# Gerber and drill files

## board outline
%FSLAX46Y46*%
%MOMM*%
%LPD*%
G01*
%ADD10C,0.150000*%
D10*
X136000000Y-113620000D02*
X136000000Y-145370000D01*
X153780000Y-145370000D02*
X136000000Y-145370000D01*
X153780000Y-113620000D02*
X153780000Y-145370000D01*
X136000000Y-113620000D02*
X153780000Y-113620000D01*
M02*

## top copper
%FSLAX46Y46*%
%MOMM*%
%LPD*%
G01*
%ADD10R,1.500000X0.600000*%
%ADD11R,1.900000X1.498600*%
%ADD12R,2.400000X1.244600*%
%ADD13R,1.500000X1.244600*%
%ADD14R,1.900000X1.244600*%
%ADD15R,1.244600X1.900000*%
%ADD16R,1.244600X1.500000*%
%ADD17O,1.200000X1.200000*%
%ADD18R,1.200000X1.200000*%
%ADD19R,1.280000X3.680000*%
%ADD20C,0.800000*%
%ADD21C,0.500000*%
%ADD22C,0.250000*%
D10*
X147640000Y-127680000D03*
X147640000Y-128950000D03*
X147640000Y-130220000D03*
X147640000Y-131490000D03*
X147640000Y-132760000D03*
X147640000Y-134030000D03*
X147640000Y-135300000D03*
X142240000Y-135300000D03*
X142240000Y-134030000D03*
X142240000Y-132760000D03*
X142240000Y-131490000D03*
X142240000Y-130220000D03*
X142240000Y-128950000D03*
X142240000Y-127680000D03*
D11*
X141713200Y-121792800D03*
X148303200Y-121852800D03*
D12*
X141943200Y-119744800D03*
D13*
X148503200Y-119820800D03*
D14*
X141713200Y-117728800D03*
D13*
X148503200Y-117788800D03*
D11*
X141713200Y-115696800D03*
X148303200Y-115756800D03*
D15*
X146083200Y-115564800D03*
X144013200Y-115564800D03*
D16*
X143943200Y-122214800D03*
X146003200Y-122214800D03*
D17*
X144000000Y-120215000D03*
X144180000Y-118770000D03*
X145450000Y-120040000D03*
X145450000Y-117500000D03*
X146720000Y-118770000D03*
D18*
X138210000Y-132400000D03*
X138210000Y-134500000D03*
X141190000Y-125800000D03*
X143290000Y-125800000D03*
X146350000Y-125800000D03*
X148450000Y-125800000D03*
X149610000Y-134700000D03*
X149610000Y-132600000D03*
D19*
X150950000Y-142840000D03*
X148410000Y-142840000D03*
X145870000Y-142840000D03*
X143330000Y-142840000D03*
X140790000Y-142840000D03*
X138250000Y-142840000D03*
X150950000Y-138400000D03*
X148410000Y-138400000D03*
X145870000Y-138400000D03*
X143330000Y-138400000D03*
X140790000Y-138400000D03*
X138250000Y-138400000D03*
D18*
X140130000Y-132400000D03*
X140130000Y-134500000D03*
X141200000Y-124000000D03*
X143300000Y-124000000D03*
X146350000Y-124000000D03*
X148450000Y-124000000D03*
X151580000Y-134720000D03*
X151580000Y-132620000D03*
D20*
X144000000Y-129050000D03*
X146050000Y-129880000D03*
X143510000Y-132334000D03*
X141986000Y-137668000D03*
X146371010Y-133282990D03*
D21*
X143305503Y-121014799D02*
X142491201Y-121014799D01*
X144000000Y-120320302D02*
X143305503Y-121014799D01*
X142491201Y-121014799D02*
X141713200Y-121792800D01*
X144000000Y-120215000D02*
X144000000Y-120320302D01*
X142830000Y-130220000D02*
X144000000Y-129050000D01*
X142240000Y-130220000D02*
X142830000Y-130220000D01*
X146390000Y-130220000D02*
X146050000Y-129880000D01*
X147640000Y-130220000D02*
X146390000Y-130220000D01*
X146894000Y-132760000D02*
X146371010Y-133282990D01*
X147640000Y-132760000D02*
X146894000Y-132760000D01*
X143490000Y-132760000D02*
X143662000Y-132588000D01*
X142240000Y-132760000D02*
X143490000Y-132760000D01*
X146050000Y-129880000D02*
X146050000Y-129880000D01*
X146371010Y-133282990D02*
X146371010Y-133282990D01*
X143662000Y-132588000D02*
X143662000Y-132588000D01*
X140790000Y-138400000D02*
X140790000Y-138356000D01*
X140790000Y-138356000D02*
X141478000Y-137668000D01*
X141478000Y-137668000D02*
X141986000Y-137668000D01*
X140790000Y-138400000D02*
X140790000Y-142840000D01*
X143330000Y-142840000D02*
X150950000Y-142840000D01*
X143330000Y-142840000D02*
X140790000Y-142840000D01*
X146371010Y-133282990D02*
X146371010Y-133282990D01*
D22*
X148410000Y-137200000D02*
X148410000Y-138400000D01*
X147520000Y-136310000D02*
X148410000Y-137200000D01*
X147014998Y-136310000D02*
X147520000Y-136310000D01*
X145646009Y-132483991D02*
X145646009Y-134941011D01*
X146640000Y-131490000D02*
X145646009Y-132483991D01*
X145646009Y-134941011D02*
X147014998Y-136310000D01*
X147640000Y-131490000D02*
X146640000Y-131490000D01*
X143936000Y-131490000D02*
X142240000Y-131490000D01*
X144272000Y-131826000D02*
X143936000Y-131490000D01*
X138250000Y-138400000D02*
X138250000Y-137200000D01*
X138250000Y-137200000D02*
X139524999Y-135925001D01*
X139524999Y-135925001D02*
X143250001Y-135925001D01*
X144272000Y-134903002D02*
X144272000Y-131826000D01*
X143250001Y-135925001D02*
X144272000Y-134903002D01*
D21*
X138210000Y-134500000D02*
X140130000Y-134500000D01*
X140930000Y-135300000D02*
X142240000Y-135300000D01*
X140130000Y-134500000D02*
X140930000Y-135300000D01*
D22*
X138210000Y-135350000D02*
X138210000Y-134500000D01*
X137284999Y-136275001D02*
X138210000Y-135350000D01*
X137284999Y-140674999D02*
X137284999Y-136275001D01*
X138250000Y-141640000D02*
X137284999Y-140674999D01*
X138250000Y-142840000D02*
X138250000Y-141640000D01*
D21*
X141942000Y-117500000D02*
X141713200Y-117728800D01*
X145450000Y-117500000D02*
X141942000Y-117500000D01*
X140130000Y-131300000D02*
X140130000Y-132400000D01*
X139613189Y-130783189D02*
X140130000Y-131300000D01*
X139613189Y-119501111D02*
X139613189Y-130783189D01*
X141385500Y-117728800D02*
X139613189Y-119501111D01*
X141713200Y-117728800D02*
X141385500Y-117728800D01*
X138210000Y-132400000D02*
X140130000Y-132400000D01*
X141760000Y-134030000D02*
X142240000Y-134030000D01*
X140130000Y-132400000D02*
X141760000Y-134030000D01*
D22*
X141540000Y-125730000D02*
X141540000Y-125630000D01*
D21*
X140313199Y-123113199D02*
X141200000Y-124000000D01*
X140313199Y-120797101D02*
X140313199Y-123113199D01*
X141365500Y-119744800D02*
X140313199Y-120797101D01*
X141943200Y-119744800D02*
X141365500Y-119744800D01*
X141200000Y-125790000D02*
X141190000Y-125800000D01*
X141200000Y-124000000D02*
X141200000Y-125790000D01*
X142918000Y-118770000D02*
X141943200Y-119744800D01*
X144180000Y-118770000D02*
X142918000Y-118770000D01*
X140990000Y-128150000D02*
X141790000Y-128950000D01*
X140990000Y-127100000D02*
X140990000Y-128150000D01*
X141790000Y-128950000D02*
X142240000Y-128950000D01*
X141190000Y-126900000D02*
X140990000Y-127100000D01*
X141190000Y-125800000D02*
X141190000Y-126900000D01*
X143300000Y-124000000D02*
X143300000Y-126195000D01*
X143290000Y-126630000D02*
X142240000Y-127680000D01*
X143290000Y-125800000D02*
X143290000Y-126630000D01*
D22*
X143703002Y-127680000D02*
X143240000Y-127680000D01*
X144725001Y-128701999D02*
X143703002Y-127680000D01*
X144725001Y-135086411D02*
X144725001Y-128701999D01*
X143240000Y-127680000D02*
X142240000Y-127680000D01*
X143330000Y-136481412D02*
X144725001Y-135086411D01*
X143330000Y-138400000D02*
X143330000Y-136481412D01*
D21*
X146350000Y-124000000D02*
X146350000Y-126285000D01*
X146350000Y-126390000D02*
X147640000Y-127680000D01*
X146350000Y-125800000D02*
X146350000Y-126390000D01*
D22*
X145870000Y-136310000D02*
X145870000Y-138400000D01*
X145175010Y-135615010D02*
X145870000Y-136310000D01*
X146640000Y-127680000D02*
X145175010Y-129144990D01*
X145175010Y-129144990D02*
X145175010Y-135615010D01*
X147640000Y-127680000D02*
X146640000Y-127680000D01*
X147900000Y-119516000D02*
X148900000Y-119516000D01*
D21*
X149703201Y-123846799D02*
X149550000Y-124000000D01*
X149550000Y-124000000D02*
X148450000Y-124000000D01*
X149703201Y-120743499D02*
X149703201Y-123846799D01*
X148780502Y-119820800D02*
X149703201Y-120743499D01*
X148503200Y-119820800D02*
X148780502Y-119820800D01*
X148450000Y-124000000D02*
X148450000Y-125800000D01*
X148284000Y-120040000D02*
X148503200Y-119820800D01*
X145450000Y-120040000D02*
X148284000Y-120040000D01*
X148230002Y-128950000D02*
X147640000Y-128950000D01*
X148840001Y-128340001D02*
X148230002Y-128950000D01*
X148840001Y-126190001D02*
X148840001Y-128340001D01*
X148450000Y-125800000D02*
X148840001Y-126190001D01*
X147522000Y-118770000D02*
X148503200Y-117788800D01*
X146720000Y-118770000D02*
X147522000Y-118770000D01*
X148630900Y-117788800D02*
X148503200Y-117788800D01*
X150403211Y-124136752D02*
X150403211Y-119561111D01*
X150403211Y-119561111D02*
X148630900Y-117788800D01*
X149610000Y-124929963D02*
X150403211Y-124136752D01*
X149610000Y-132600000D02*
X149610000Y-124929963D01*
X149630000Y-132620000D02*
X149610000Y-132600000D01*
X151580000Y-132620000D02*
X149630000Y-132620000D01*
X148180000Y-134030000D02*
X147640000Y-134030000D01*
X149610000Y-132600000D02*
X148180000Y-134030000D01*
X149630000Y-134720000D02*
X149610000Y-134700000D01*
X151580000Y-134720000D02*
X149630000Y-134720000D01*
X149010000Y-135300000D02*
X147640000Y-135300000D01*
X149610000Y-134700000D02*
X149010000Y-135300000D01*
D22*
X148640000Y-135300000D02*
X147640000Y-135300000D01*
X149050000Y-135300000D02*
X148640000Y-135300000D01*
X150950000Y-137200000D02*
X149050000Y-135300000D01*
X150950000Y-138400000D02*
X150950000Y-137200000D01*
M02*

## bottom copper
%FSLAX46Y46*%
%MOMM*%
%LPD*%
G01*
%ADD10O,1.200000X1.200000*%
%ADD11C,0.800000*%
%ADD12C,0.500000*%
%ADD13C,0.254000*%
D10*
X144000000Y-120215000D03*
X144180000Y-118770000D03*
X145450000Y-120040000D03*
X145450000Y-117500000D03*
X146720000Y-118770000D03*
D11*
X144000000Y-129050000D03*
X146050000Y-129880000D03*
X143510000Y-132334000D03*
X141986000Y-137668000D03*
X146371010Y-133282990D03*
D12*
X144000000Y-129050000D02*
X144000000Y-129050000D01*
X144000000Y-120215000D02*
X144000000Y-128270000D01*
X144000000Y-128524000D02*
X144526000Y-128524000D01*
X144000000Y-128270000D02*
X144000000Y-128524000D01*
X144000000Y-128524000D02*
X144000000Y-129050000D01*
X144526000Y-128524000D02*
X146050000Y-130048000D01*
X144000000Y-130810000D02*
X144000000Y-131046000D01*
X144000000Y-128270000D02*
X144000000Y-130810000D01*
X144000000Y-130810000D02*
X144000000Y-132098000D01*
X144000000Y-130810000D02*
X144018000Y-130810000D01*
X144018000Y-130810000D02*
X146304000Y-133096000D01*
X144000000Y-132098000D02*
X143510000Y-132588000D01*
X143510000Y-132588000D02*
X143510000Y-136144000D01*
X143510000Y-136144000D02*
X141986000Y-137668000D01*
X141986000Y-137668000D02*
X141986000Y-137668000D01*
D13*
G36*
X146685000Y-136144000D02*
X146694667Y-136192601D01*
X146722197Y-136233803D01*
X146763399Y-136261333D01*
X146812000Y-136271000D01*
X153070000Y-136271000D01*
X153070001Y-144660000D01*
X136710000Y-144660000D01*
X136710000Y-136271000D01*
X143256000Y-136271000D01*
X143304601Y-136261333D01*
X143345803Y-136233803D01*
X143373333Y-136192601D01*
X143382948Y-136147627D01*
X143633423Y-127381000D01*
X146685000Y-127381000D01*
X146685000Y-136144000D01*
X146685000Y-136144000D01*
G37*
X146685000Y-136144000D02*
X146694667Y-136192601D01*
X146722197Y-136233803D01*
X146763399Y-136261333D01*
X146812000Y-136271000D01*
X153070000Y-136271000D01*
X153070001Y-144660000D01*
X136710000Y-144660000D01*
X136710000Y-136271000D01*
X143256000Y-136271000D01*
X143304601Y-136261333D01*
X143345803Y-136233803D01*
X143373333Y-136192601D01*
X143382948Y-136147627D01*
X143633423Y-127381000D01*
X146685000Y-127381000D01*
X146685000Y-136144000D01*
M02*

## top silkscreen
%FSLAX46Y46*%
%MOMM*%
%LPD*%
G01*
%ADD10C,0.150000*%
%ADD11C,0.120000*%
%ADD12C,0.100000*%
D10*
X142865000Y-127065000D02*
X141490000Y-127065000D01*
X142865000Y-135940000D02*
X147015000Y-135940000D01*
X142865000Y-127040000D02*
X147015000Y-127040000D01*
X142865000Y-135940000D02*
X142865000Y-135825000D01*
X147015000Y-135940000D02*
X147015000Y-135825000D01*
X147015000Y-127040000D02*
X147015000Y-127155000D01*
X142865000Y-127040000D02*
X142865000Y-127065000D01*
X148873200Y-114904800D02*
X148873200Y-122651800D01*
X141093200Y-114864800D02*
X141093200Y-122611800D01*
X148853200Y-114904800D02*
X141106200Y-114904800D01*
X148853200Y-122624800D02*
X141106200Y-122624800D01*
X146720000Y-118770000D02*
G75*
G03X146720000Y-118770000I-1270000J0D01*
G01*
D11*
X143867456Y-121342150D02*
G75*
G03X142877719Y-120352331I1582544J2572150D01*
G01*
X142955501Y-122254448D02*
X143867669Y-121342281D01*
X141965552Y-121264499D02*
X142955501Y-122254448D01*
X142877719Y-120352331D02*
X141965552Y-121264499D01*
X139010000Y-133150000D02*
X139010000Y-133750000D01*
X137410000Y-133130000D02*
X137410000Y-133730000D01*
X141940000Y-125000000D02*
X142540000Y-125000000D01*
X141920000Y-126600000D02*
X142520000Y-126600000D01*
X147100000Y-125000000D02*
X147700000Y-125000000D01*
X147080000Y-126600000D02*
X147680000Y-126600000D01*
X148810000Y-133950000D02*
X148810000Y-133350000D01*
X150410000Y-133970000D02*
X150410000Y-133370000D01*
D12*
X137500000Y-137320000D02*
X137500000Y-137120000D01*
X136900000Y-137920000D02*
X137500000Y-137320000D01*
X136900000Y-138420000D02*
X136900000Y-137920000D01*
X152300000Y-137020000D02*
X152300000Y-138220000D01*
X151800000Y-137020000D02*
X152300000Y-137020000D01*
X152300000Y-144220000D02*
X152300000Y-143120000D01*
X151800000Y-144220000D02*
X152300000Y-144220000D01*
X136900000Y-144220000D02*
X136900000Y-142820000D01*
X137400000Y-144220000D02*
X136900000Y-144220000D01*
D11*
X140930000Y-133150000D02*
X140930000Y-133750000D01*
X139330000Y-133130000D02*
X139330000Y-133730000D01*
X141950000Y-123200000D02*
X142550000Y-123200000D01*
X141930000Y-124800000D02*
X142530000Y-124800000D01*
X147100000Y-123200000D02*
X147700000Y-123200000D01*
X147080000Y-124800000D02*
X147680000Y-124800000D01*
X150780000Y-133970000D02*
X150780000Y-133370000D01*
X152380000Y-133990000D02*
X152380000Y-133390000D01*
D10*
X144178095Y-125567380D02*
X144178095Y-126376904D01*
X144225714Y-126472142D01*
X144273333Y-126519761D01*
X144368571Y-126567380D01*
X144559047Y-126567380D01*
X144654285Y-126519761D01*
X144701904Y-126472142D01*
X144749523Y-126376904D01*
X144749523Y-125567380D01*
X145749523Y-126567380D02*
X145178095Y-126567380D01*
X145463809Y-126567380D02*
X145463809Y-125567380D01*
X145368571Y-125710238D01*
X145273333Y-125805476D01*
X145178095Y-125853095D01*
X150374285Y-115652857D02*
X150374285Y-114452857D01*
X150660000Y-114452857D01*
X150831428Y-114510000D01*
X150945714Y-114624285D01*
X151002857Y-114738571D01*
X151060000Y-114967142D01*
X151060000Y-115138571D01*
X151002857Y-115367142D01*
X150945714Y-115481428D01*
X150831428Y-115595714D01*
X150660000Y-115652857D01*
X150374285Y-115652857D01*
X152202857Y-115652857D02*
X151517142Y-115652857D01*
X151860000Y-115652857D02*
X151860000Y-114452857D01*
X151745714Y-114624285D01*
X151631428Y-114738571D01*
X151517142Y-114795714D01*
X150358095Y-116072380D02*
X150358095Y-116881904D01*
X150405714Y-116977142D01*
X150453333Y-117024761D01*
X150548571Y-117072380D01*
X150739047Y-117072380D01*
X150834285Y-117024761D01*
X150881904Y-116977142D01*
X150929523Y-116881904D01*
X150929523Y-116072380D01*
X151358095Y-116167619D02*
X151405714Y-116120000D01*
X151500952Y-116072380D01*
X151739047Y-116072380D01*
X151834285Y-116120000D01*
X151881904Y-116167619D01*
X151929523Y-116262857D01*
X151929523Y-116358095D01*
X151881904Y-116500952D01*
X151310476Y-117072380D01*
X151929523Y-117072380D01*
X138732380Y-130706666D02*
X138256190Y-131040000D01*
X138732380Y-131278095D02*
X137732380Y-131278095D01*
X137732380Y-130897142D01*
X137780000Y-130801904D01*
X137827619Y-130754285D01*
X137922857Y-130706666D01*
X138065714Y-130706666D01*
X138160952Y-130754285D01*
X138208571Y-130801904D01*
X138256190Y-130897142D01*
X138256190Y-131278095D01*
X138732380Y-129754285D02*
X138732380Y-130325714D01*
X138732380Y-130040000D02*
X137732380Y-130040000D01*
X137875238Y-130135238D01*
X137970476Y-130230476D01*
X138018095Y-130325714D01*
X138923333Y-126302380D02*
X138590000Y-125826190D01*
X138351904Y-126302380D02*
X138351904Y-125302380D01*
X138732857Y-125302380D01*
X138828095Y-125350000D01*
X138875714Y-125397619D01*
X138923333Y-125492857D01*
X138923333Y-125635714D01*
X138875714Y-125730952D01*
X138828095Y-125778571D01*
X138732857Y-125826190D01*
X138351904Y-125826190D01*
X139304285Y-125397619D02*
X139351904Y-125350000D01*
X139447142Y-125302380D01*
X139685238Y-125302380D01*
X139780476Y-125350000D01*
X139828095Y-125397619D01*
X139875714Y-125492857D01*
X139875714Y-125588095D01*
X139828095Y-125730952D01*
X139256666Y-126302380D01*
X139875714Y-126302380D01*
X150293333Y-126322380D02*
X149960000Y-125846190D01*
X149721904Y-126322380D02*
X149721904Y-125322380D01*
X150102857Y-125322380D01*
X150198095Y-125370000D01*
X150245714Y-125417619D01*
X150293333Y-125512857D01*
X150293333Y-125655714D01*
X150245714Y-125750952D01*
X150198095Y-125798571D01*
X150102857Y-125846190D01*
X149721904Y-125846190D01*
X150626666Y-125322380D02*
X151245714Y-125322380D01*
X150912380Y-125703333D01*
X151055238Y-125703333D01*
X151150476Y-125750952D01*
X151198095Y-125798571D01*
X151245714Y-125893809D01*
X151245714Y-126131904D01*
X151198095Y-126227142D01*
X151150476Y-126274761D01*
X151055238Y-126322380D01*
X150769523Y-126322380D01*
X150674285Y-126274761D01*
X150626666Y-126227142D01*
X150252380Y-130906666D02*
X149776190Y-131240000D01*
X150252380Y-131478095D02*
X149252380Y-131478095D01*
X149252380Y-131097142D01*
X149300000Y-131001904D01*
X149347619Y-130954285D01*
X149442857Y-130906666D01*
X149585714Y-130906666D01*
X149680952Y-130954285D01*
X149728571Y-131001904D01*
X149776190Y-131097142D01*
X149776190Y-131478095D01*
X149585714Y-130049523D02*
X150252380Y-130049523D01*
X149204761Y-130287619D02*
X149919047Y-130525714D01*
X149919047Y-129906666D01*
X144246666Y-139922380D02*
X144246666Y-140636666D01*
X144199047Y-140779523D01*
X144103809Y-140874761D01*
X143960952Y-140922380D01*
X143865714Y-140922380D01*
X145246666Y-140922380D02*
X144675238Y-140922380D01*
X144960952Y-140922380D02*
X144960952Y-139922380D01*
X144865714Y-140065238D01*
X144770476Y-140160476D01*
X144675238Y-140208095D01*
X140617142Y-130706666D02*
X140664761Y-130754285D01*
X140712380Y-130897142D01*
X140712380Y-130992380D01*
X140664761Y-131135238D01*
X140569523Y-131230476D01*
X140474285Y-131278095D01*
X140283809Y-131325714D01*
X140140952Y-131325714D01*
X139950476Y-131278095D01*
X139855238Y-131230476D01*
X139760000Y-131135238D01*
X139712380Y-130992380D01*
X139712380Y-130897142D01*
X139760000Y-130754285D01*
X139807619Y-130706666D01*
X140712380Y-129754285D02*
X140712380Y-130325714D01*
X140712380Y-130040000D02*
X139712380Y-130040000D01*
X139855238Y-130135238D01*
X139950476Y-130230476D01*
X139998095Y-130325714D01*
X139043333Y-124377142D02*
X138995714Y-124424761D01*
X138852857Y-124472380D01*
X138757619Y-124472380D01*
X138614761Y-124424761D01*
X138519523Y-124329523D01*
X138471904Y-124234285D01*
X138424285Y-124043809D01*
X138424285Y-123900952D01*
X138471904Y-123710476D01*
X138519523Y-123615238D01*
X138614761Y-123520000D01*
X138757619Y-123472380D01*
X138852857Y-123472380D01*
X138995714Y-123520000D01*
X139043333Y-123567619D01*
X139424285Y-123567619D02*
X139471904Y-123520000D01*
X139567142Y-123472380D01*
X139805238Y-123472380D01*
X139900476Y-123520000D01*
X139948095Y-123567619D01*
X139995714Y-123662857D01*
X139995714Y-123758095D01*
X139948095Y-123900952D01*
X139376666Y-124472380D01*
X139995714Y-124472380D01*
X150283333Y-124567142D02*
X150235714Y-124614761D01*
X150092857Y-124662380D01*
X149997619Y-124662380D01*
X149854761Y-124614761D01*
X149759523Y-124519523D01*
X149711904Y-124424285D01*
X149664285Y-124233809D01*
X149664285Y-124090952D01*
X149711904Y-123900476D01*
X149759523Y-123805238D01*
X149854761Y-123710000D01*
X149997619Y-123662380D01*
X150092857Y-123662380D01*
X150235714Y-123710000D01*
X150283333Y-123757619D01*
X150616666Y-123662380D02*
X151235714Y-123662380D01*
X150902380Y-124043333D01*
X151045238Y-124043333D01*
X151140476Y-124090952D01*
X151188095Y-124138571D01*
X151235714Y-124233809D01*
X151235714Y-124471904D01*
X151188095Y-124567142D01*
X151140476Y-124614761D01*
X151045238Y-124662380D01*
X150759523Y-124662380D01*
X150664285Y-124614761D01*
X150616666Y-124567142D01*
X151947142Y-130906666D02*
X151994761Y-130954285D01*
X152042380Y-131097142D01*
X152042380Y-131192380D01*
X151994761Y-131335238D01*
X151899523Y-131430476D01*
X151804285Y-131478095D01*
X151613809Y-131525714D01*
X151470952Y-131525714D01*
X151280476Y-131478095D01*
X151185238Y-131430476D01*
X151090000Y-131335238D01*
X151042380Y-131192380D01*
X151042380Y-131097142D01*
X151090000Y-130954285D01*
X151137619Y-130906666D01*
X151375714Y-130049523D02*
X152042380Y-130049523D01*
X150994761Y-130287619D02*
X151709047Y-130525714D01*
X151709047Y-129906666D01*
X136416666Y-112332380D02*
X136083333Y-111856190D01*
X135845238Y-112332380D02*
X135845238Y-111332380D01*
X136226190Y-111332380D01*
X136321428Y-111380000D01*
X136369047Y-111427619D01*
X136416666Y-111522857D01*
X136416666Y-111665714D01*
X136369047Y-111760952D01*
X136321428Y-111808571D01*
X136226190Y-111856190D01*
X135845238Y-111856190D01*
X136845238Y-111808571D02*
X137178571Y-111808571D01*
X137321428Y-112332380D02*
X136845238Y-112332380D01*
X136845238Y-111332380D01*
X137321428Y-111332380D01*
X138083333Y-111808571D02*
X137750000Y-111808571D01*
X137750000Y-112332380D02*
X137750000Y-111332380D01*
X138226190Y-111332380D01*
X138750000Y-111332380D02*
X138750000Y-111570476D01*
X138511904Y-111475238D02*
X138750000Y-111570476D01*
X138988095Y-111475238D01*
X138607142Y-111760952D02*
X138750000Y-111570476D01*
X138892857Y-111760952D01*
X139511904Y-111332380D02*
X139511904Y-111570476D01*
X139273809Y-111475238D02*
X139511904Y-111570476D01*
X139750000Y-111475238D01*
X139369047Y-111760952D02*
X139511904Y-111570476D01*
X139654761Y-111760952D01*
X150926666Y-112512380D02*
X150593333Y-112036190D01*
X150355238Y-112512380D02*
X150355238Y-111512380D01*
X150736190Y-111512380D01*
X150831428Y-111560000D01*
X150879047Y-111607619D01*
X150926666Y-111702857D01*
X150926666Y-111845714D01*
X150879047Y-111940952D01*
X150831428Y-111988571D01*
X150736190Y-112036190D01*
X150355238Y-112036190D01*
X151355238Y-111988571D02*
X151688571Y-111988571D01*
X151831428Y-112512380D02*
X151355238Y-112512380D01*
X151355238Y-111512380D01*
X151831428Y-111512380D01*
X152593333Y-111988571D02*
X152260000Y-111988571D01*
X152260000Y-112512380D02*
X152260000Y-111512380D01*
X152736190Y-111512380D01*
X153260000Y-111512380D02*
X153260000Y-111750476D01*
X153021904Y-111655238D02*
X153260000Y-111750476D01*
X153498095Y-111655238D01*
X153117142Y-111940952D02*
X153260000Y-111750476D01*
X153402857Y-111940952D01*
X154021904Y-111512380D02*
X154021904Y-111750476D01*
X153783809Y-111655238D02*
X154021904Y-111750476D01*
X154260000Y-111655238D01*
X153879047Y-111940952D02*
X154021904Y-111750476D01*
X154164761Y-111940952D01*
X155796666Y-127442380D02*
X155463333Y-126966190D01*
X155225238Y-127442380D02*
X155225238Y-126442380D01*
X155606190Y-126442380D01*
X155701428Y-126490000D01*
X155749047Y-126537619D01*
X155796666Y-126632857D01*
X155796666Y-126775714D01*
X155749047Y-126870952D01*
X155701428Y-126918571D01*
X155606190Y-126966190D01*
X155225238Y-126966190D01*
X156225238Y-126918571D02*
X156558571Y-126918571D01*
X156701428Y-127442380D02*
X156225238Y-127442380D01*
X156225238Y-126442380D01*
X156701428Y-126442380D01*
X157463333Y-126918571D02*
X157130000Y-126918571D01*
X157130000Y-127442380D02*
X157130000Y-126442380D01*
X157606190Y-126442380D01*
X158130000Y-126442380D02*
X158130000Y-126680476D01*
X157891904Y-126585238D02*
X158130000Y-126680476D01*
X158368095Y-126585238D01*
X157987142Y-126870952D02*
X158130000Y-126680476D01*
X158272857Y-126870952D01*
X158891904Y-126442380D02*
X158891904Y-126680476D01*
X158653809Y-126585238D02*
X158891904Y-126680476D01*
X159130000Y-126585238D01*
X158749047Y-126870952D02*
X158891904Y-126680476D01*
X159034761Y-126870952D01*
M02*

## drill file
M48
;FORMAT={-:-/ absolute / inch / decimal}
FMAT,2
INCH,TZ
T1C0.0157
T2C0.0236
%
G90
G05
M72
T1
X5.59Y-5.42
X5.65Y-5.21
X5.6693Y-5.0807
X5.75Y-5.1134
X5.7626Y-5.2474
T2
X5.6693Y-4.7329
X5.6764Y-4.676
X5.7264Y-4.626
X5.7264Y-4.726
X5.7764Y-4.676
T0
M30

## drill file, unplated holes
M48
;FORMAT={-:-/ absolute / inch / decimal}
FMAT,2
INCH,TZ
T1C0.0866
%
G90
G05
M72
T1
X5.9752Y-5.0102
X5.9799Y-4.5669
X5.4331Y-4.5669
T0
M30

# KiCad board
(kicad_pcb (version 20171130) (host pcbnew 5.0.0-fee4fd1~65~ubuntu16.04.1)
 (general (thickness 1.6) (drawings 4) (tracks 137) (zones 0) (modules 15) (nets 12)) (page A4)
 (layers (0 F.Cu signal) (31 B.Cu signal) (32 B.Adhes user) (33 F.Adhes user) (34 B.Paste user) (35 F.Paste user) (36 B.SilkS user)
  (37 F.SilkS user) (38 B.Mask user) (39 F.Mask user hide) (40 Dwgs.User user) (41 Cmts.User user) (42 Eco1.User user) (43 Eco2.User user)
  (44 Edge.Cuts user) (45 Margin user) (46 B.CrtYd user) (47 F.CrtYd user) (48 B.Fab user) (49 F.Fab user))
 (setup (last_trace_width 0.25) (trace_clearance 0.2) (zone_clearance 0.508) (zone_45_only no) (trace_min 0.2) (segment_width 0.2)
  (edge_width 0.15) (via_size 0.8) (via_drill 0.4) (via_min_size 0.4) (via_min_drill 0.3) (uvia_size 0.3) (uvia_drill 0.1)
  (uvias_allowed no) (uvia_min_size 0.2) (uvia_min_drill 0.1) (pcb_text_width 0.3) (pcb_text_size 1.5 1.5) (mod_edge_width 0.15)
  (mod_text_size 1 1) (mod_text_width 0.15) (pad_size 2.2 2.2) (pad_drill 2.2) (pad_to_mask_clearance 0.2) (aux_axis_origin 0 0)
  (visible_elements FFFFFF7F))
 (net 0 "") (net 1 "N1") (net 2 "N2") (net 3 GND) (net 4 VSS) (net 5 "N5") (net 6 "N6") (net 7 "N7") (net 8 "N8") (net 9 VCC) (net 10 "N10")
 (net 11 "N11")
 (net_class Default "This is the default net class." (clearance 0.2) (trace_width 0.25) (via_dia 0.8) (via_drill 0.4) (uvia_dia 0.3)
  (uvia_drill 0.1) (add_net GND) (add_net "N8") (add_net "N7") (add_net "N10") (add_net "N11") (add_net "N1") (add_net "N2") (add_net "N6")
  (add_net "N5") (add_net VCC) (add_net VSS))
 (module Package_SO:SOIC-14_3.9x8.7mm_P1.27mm (layer F.Cu) (at 144.94 131.49)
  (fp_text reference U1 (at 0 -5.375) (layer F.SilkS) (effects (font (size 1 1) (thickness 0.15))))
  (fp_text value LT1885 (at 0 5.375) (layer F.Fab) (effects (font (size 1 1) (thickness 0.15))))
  (fp_line (start -2.075 -4.425) (end -3.45 -4.425) (layer F.SilkS) (width 0.15))
  (fp_line (start -2.075 4.45) (end 2.075 4.45) (layer F.SilkS) (width 0.15))
  (fp_line (start -2.075 -4.45) (end 2.075 -4.45) (layer F.SilkS) (width 0.15))
  (fp_line (start -2.075 4.45) (end -2.075 4.335) (layer F.SilkS) (width 0.15))
  (fp_line (start 2.075 4.45) (end 2.075 4.335) (layer F.SilkS) (width 0.15))
  (fp_line (start 2.075 -4.45) (end 2.075 -4.335) (layer F.SilkS) (width 0.15))
  (fp_line (start -2.075 -4.45) (end -2.075 -4.425) (layer F.SilkS) (width 0.15))
  (pad 14 smd rect (at 2.7 -3.81) (size 1.5 0.6) (layers F.Cu F.Paste F.Mask) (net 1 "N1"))
  (pad 13 smd rect (at 2.7 -2.54) (size 1.5 0.6) (layers F.Cu F.Paste F.Mask) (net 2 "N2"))
  (pad 12 smd rect (at 2.7 -1.27) (size 1.5 0.6) (layers F.Cu F.Paste F.Mask) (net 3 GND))
  (pad 11 smd rect (at 2.7 0) (size 1.5 0.6) (layers F.Cu F.Paste F.Mask) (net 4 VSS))
  (pad 10 smd rect (at 2.7 1.27) (size 1.5 0.6) (layers F.Cu F.Paste F.Mask) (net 3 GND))
  (pad 9 smd rect (at 2.7 2.54) (size 1.5 0.6) (layers F.Cu F.Paste F.Mask) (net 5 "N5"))
  (pad 8 smd rect (at 2.7 3.81) (size 1.5 0.6) (layers F.Cu F.Paste F.Mask) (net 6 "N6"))
  (pad 7 smd rect (at -2.7 3.81) (size 1.5 0.6) (layers F.Cu F.Paste F.Mask) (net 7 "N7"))
  (pad 6 smd rect (at -2.7 2.54) (size 1.5 0.6) (layers F.Cu F.Paste F.Mask) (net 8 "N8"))
  (pad 5 smd rect (at -2.7 1.27) (size 1.5 0.6) (layers F.Cu F.Paste F.Mask) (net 3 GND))
  (pad 4 smd rect (at -2.7 0) (size 1.5 0.6) (layers F.Cu F.Paste F.Mask) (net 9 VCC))
  (pad 3 smd rect (at -2.7 -1.27) (size 1.5 0.6) (layers F.Cu F.Paste F.Mask) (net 3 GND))
  (pad 2 smd rect (at -2.7 -2.54) (size 1.5 0.6) (layers F.Cu F.Paste F.Mask) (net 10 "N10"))
  (pad 1 smd rect (at -2.7 -3.81) (size 1.5 0.6) (layers F.Cu F.Paste F.Mask) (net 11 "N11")))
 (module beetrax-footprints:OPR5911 (layer F.Cu) (at 148.7932 117.1448 270)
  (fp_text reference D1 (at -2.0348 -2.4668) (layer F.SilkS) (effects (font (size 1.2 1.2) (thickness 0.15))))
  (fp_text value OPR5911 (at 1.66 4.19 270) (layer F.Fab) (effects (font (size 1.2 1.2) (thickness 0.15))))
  (fp_line (start -2.24 -0.08) (end 5.507 -0.08) (layer F.SilkS) (width 0.15))
  (fp_line (start -2.28 7.7) (end 5.467 7.7) (layer F.SilkS) (width 0.15))
  (fp_line (start -2.24 -0.06) (end -2.24 7.687) (layer F.SilkS) (width 0.15))
  (fp_line (start 5.48 -0.06) (end 5.48 7.687) (layer F.SilkS) (width 0.15))
  (pad 2 smd rect (at 4.648 7.08 270) (size 1.4986 1.9) (layers F.Cu F.Paste F.Mask) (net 3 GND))
  (pad 5 smd rect (at 4.708 0.49 270) (size 1.4986 1.9) (layers F.Cu F.Paste F.Mask))
  (pad 1 smd rect (at 2.6 6.85 270) (size 1.2446 2.4) (layers F.Cu F.Paste F.Mask) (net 10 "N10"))
  (pad 6 smd rect (at 2.676 0.29 270) (size 1.2446 1.5) (layers F.Cu F.Paste F.Mask) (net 2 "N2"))
  (pad 12 smd rect (at 0.584 7.08 270) (size 1.2446 1.9) (layers F.Cu F.Paste F.Mask) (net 8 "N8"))
  (pad 7 smd rect (at 0.644 0.29 270) (size 1.2446 1.5) (layers F.Cu F.Paste F.Mask) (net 5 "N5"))
  (pad 11 smd rect (at -1.448 7.08 270) (size 1.4986 1.9) (layers F.Cu F.Paste F.Mask))
  (pad 8 smd rect (at -1.388 0.49 270) (size 1.4986 1.9) (layers F.Cu F.Paste F.Mask))
  (pad 9 smd rect (at -1.58 2.71 270) (size 1.9 1.2446) (layers F.Cu F.Paste F.Mask))
  (pad 10 smd rect (at -1.58 4.78 270) (size 1.9 1.2446) (layers F.Cu F.Paste F.Mask))
  (pad 3 smd rect (at 5.07 4.85 270) (size 1.5 1.2446) (layers F.Cu F.Paste F.Mask))
  (pad 4 smd rect (at 5.07 2.79 270) (size 1.5 1.2446) (layers F.Cu F.Paste F.Mask)))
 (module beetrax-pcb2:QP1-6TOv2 (layer F.Cu) (at 145.45 120.04 90)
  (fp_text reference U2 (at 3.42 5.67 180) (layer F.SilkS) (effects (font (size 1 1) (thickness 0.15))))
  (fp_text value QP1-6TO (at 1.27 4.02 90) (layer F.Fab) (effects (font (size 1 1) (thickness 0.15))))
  (fp_circle (center 1.27 0) (end 1.27 1.27) (layer F.SilkS) (width 0.15))
  (fp_arc (start 1.27 0) (end -0.312331 -2.572281) (angle 333.2) (layer F.SilkS) (width 0.12))
  (fp_line (start -2.214448 -2.494499) (end -1.302281 -1.582331) (layer F.SilkS) (width 0.12))
  (fp_line (start -1.224499 -3.484448) (end -2.214448 -2.494499) (layer F.SilkS) (width 0.12))
  (fp_line (start -0.312331 -2.572281) (end -1.224499 -3.484448) (layer F.SilkS) (width 0.12))
  (pad 5 thru_hole oval (at -0.175 -1.45 90) (size 1.2 1.2) (drill 0.6) (layers *.Cu *.Mask) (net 3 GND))
  (pad 1 thru_hole oval (at 1.27 -1.27 90) (size 1.2 1.2) (drill 0.6) (layers *.Cu *.Mask) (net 10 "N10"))
  (pad 4 thru_hole oval (at 0 0 90) (size 1.2 1.2) (drill 0.6) (layers *.Cu *.Mask) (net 2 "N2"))
  (pad 2 thru_hole oval (at 2.54 0 90) (size 1.2 1.2) (drill 0.6) (layers *.Cu *.Mask) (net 8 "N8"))
  (pad 3 thru_hole oval (at 1.27 1.27 90) (size 1.2 1.2) (drill 0.6) (layers *.Cu *.Mask) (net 5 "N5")))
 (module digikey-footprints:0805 (layer F.Cu) (at 138.21 133.45 270)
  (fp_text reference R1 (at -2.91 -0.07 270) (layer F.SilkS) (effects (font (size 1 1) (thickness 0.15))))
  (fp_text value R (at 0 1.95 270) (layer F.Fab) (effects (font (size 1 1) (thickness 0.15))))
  (fp_line (start -0.3 -0.8) (end 0.3 -0.8) (layer F.SilkS) (width 0.12))
  (fp_line (start -0.32 0.8) (end 0.28 0.8) (layer F.SilkS) (width 0.12))
  (pad 1 smd rect (at -1.05 0 270) (size 1.2 1.2) (layers F.Cu F.Paste F.Mask) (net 8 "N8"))
  (pad 2 smd rect (at 1.05 0 270) (size 1.2 1.2) (layers F.Cu F.Paste F.Mask) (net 7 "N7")))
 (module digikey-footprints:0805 (layer F.Cu) (at 142.24 125.8)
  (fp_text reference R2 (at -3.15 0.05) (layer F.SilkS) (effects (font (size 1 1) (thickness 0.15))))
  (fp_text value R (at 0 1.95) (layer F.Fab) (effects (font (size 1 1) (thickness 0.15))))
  (fp_line (start -0.3 -0.8) (end 0.3 -0.8) (layer F.SilkS) (width 0.12))
  (fp_line (start -0.32 0.8) (end 0.28 0.8) (layer F.SilkS) (width 0.12))
  (pad 1 smd rect (at -1.05 0) (size 1.2 1.2) (layers F.Cu F.Paste F.Mask) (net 10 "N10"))
  (pad 2 smd rect (at 1.05 0) (size 1.2 1.2) (layers F.Cu F.Paste F.Mask) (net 11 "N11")))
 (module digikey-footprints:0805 (layer F.Cu) (at 147.4 125.8)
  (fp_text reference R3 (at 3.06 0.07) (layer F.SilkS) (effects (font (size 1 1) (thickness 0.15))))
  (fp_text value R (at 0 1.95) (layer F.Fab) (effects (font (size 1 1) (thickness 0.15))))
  (fp_line (start -0.3 -0.8) (end 0.3 -0.8) (layer F.SilkS) (width 0.12))
  (fp_line (start -0.32 0.8) (end 0.28 0.8) (layer F.SilkS) (width 0.12))
  (pad 1 smd rect (at -1.05 0) (size 1.2 1.2) (layers F.Cu F.Paste F.Mask) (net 1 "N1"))
  (pad 2 smd rect (at 1.05 0) (size 1.2 1.2) (layers F.Cu F.Paste F.Mask) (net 2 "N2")))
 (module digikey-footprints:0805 (layer F.Cu) (at 149.61 133.65 90)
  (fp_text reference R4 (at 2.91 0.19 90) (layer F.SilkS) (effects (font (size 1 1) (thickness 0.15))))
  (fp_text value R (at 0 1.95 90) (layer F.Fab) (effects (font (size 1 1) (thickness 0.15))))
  (fp_line (start -0.3 -0.8) (end 0.3 -0.8) (layer F.SilkS) (width 0.12))
  (fp_line (start -0.32 0.8) (end 0.28 0.8) (layer F.SilkS) (width 0.12))
  (pad 1 smd rect (at -1.05 0 90) (size 1.2 1.2) (layers F.Cu F.Paste F.Mask) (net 6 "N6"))
  (pad 2 smd rect (at 1.05 0 90) (size 1.2 1.2) (layers F.Cu F.Paste F.Mask) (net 5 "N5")))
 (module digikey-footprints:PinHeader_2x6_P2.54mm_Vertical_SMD (layer F.Cu) (at 144.6 140.62)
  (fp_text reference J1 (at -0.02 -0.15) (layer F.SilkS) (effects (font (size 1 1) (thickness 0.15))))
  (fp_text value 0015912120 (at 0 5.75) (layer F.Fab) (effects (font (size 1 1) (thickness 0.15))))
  (fp_line (start -7.1 -3.3) (end -7.1 -3.5) (layer F.SilkS) (width 0.1))
  (fp_line (start -7.7 -2.7) (end -7.1 -3.3) (layer F.SilkS) (width 0.1))
  (fp_line (start -7.7 -2.2) (end -7.7 -2.7) (layer F.SilkS) (width 0.1))
  (fp_line (start 7.7 -3.6) (end 7.7 -2.4) (layer F.SilkS) (width 0.1))
  (fp_line (start 7.2 -3.6) (end 7.7 -3.6) (layer F.SilkS) (width 0.1))
  (fp_line (start 7.7 3.6) (end 7.7 2.5) (layer F.SilkS) (width 0.1))
  (fp_line (start 7.2 3.6) (end 7.7 3.6) (layer F.SilkS) (width 0.1))
  (fp_line (start -7.7 3.6) (end -7.7 2.2) (layer F.SilkS) (width 0.1))
  (fp_line (start -7.2 3.6) (end -7.7 3.6) (layer F.SilkS) (width 0.1))
  (pad 12 smd rect (at 6.35 2.22) (size 1.28 3.68) (layers F.Cu F.Paste F.Mask) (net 3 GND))
  (pad 11 smd rect (at 3.81 2.22) (size 1.28 3.68) (layers F.Cu F.Paste F.Mask) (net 3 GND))
  (pad 10 smd rect (at 1.27 2.22) (size 1.28 3.68) (layers F.Cu F.Paste F.Mask) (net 3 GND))
  (pad 9 smd rect (at -1.27 2.22) (size 1.28 3.68) (layers F.Cu F.Paste F.Mask) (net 3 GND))
  (pad 8 smd rect (at -3.81 2.22) (size 1.28 3.68) (layers F.Cu F.Paste F.Mask) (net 3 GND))
  (pad 7 smd rect (at -6.35 2.22) (size 1.28 3.68) (layers F.Cu F.Paste F.Mask) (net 7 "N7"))
  (pad 6 smd rect (at 6.35 -2.22) (size 1.28 3.68) (layers F.Cu F.Paste F.Mask) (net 6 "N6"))
  (pad 5 smd rect (at 3.81 -2.22) (size 1.28 3.68) (layers F.Cu F.Paste F.Mask) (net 4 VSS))
  (pad 4 smd rect (at 1.27 -2.22) (size 1.28 3.68) (layers F.Cu F.Paste F.Mask) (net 1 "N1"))
  (pad 3 smd rect (at -1.27 -2.22) (size 1.28 3.68) (layers F.Cu F.Paste F.Mask) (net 11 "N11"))
  (pad 2 smd rect (at -3.81 -2.22) (size 1.28 3.68) (layers F.Cu F.Paste F.Mask) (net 3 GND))
  (pad 1 smd rect (at -6.35 -2.22) (size 1.28 3.68) (layers F.Cu F.Paste F.Mask) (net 9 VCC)))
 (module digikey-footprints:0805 (layer F.Cu) (at 140.13 133.45 270)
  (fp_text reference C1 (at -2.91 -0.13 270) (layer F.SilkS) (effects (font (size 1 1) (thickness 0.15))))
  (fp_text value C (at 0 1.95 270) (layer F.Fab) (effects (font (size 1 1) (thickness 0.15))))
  (fp_line (start -0.3 -0.8) (end 0.3 -0.8) (layer F.SilkS) (width 0.12))
  (fp_line (start -0.32 0.8) (end 0.28 0.8) (layer F.SilkS) (width 0.12))
  (pad 1 smd rect (at -1.05 0 270) (size 1.2 1.2) (layers F.Cu F.Paste F.Mask) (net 8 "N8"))
  (pad 2 smd rect (at 1.05 0 270) (size 1.2 1.2) (layers F.Cu F.Paste F.Mask) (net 7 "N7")))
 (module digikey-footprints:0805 (layer F.Cu) (at 142.25 124)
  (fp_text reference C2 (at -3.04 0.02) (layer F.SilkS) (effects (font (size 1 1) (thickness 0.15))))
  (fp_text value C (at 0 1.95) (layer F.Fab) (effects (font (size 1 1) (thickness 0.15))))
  (fp_line (start -0.3 -0.8) (end 0.3 -0.8) (layer F.SilkS) (width 0.12))
  (fp_line (start -0.32 0.8) (end 0.28 0.8) (layer F.SilkS) (width 0.12))
  (pad 1 smd rect (at -1.05 0) (size 1.2 1.2) (layers F.Cu F.Paste F.Mask) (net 10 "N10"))
  (pad 2 smd rect (at 1.05 0) (size 1.2 1.2) (layers F.Cu F.Paste F.Mask) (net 11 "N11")))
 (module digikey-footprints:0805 (layer F.Cu) (at 147.4 124)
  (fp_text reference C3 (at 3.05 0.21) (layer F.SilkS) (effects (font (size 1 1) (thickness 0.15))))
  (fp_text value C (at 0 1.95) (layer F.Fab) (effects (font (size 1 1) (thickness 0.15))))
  (fp_line (start -0.3 -0.8) (end 0.3 -0.8) (layer F.SilkS) (width 0.12))
  (fp_line (start -0.32 0.8) (end 0.28 0.8) (layer F.SilkS) (width 0.12))
  (pad 1 smd rect (at -1.05 0) (size 1.2 1.2) (layers F.Cu F.Paste F.Mask) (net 1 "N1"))
  (pad 2 smd rect (at 1.05 0) (size 1.2 1.2) (layers F.Cu F.Paste F.Mask) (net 2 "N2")))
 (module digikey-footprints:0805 (layer F.Cu) (at 151.58 133.67 90)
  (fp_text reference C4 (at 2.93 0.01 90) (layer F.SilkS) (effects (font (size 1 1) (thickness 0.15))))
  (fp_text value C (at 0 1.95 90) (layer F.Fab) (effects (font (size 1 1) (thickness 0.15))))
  (fp_line (start -0.3 -0.8) (end 0.3 -0.8) (layer F.SilkS) (width 0.12))
  (fp_line (start -0.32 0.8) (end 0.28 0.8) (layer F.SilkS) (width 0.12))
  (pad 1 smd rect (at -1.05 0 90) (size 1.2 1.2) (layers F.Cu F.Paste F.Mask) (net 6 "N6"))
  (pad 2 smd rect (at 1.05 0 90) (size 1.2 1.2) (layers F.Cu F.Paste F.Mask) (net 5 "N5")))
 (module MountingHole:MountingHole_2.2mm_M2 (layer F.Cu) (at 138 116)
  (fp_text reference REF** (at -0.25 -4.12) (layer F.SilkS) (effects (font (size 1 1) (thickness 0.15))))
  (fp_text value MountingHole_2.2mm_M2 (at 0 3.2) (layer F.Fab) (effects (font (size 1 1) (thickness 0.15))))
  (pad 1 np_thru_hole circle (at 0 0) (size 2.2 2.2) (drill 2.2) (layers *.Cu *.Mask)))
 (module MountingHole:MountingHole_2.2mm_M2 (layer F.Cu) (at 151.89 116)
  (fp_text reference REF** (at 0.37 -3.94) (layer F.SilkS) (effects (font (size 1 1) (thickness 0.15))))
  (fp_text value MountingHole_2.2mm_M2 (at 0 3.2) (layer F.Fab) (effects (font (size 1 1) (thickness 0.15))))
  (pad 1 np_thru_hole circle (at 0 0) (size 2.2 2.2) (drill 2.2) (layers *.Cu *.Mask)))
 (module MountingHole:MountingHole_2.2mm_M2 (layer F.Cu) (at 151.77 127.26)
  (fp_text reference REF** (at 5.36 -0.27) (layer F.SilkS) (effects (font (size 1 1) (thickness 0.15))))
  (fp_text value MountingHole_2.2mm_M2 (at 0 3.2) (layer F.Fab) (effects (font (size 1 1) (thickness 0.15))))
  (pad 1 np_thru_hole circle (at 0 0) (size 2.2 2.2) (drill 2.2) (layers *.Cu *.Mask)))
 (gr_line (start 136 113.62) (end 136 145.37) (layer Edge.Cuts) (width 0.15))
 (gr_line (start 153.78 145.37) (end 136 145.37) (layer Edge.Cuts) (width 0.15))
 (gr_line (start 153.78 113.62) (end 153.78 145.37) (layer Edge.Cuts) (width 0.15))
 (gr_line (start 136 113.62) (end 153.78 113.62) (layer Edge.Cuts) (width 0.15))
 (segment (start 143.305503 121.014799) (end 142.491201 121.014799) (width 0.5) (layer F.Cu) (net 3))
 (segment (start 144 120.320302) (end 143.305503 121.014799) (width 0.5) (layer F.Cu) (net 3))
 (segment (start 142.491201 121.014799) (end 141.7132 121.7928) (width 0.5) (layer F.Cu) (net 3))
 (segment (start 144 120.215) (end 144 120.320302) (width 0.5) (layer F.Cu) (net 3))
 (segment (start 144 129.05) (end 144 129.05) (width 0.5) (layer B.Cu) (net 3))
 (via (at 144 129.05) (size 0.8) (drill 0.4) (layers F.Cu B.Cu) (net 3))
 (segment (start 142.83 130.22) (end 144 129.05) (width 0.5) (layer F.Cu) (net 3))
 (segment (start 142.24 130.22) (end 142.83 130.22) (width 0.5) (layer F.Cu) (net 3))
 (segment (start 146.39 130.22) (end 146.05 129.88) (width 0.5) (layer F.Cu) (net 3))
 (segment (start 147.64 130.22) (end 146.39 130.22) (width 0.5) (layer F.Cu) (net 3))
 (segment (start 146.894 132.76) (end 146.37101 133.28299) (width 0.5) (layer F.Cu) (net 3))
 (segment (start 147.64 132.76) (end 146.894 132.76) (width 0.5) (layer F.Cu) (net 3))
 (segment (start 143.49 132.76) (end 143.662 132.588) (width 0.5) (layer F.Cu) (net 3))
 (segment (start 142.24 132.76) (end 143.49 132.76) (width 0.5) (layer F.Cu) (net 3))
 (segment (start 144 120.215) (end 144 128.27) (width 0.5) (layer B.Cu) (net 3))
 (segment (start 144 128.524) (end 144.526 128.524) (width 0.5) (layer B.Cu) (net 3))
 (segment (start 144 128.27) (end 144 128.524) (width 0.5) (layer B.Cu) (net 3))
 (segment (start 144 128.524) (end 144 129.05) (width 0.5) (layer B.Cu) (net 3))
 (segment (start 144.526 128.524) (end 146.05 130.048) (width 0.5) (layer B.Cu) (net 3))
 (segment (start 144 130.81) (end 144 131.046) (width 0.5) (layer B.Cu) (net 3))
 (segment (start 144 128.27) (end 144 130.81) (width 0.5) (layer B.Cu) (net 3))
 (segment (start 144 130.81) (end 144 132.098) (width 0.5) (layer B.Cu) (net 3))
 (segment (start 144 130.81) (end 144.018 130.81) (width 0.5) (layer B.Cu) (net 3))
 (segment (start 144.018 130.81) (end 146.304 133.096) (width 0.5) (layer B.Cu) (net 3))
 (segment (start 144 132.098) (end 143.51 132.588) (width 0.5) (layer B.Cu) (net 3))
 (segment (start 143.51 132.588) (end 143.51 136.144) (width 0.5) (layer B.Cu) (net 3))
 (segment (start 143.51 136.144) (end 141.986 137.668) (width 0.5) (layer B.Cu) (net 3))
 (segment (start 146.05 129.88) (end 146.05 129.88) (width 0.5) (layer F.Cu) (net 3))
 (via (at 146.05 129.88) (size 0.8) (drill 0.4) (layers F.Cu B.Cu) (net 3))
 (segment (start 146.37101 133.28299) (end 146.37101 133.28299) (width 0.5) (layer F.Cu) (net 3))
 (segment (start 143.662 132.588) (end 143.662 132.588) (width 0.5) (layer F.Cu) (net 3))
 (via (at 143.51 132.334) (size 0.8) (drill 0.4) (layers F.Cu B.Cu) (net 3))
 (segment (start 140.79 138.4) (end 140.79 138.356) (width 0.5) (layer F.Cu) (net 3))
 (segment (start 140.79 138.356) (end 141.478 137.668) (width 0.5) (layer F.Cu) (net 3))
 (segment (start 141.478 137.668) (end 141.986 137.668) (width 0.5) (layer F.Cu) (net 3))
 (segment (start 141.986 137.668) (end 141.986 137.668) (width 0.5) (layer B.Cu) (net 3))
 (via (at 141.986 137.668) (size 0.8) (drill 0.4) (layers F.Cu B.Cu) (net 3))
 (segment (start 140.79 138.4) (end 140.79 142.84) (width 0.5) (layer F.Cu) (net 3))
 (segment (start 143.33 142.84) (end 150.95 142.84) (width 0.5) (layer F.Cu) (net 3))
 (segment (start 143.33 142.84) (end 140.79 142.84) (width 0.5) (layer F.Cu) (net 3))
 (segment (start 146.37101 133.28299) (end 146.37101 133.28299) (width 0.5) (layer F.Cu) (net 3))
 (via (at 146.37101 133.28299) (size 0.8) (drill 0.4) (layers F.Cu B.Cu) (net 3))
 (segment (start 148.41 137.2) (end 148.41 138.4) (width 0.25) (layer F.Cu) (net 4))
 (segment (start 147.52 136.31) (end 148.41 137.2) (width 0.25) (layer F.Cu) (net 4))
 (segment (start 147.014998 136.31) (end 147.52 136.31) (width 0.25) (layer F.Cu) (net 4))
 (segment (start 145.646009 132.483991) (end 145.646009 134.941011) (width 0.25) (layer F.Cu) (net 4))
 (segment (start 146.64 131.49) (end 145.646009 132.483991) (width 0.25) (layer F.Cu) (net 4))
 (segment (start 145.646009 134.941011) (end 147.014998 136.31) (width 0.25) (layer F.Cu) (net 4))
 (segment (start 147.64 131.49) (end 146.64 131.49) (width 0.25) (layer F.Cu) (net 4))
 (segment (start 143.936 131.49) (end 142.24 131.49) (width 0.25) (layer F.Cu) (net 9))
 (segment (start 144.272 131.826) (end 143.936 131.49) (width 0.25) (layer F.Cu) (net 9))
 (segment (start 138.25 138.4) (end 138.25 137.2) (width 0.25) (layer F.Cu) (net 9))
 (segment (start 138.25 137.2) (end 139.524999 135.925001) (width 0.25) (layer F.Cu) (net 9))
 (segment (start 139.524999 135.925001) (end 143.250001 135.925001) (width 0.25) (layer F.Cu) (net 9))
 (segment (start 144.272 134.903002) (end 144.272 131.826) (width 0.25) (layer F.Cu) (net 9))
 (segment (start 143.250001 135.925001) (end 144.272 134.903002) (width 0.25) (layer F.Cu) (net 9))
 (segment (start 138.21 134.5) (end 140.13 134.5) (width 0.5) (layer F.Cu) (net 7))
 (segment (start 140.93 135.3) (end 142.24 135.3) (width 0.5) (layer F.Cu) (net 7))
 (segment (start 140.13 134.5) (end 140.93 135.3) (width 0.5) (layer F.Cu) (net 7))
 (segment (start 138.21 135.35) (end 138.21 134.5) (width 0.25) (layer F.Cu) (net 7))
 (segment (start 137.284999 136.275001) (end 138.21 135.35) (width 0.25) (layer F.Cu) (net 7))
 (segment (start 137.284999 140.674999) (end 137.284999 136.275001) (width 0.25) (layer F.Cu) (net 7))
 (segment (start 138.25 141.64) (end 137.284999 140.674999) (width 0.25) (layer F.Cu) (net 7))
 (segment (start 138.25 142.84) (end 138.25 141.64) (width 0.25) (layer F.Cu) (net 7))
 (segment (start 141.942 117.5) (end 141.7132 117.7288) (width 0.5) (layer F.Cu) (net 8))
 (segment (start 145.45 117.5) (end 141.942 117.5) (width 0.5) (layer F.Cu) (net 8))
 (segment (start 140.13 131.3) (end 140.13 132.4) (width 0.5) (layer F.Cu) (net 8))
 (segment (start 139.613189 130.783189) (end 140.13 131.3) (width 0.5) (layer F.Cu) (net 8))
 (segment (start 139.613189 119.501111) (end 139.613189 130.783189) (width 0.5) (layer F.Cu) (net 8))
 (segment (start 141.3855 117.7288) (end 139.613189 119.501111) (width 0.5) (layer F.Cu) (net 8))
 (segment (start 141.7132 117.7288) (end 141.3855 117.7288) (width 0.5) (layer F.Cu) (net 8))
 (segment (start 138.21 132.4) (end 140.13 132.4) (width 0.5) (layer F.Cu) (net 8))
 (segment (start 141.76 134.03) (end 142.24 134.03) (width 0.5) (layer F.Cu) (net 8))
 (segment (start 140.13 132.4) (end 141.76 134.03) (width 0.5) (layer F.Cu) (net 8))
 (segment (start 141.54 125.73) (end 141.54 125.63) (width 0.25) (layer F.Cu) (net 10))
 (segment (start 140.313199 123.113199) (end 141.2 124) (width 0.5) (layer F.Cu) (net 10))
 (segment (start 140.313199 120.797101) (end 140.313199 123.113199) (width 0.5) (layer F.Cu) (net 10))
 (segment (start 141.3655 119.7448) (end 140.313199 120.797101) (width 0.5) (layer F.Cu) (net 10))
 (segment (start 141.9432 119.7448) (end 141.3655 119.7448) (width 0.5) (layer F.Cu) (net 10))
 (segment (start 141.2 125.79) (end 141.19 125.8) (width 0.5) (layer F.Cu) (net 10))
 (segment (start 141.2 124) (end 141.2 125.79) (width 0.5) (layer F.Cu) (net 10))
 (segment (start 142.918 118.77) (end 141.9432 119.7448) (width 0.5) (layer F.Cu) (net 10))
 (segment (start 144.18 118.77) (end 142.918 118.77) (width 0.5) (layer F.Cu) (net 10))
 (segment (start 140.99 128.15) (end 141.79 128.95) (width 0.5) (layer F.Cu) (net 10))
 (segment (start 140.99 127.1) (end 140.99 128.15) (width 0.5) (layer F.Cu) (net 10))
 (segment (start 141.79 128.95) (end 142.24 128.95) (width 0.5) (layer F.Cu) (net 10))
 (segment (start 141.19 126.9) (end 140.99 127.1) (width 0.5) (layer F.Cu) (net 10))
 (segment (start 141.19 125.8) (end 141.19 126.9) (width 0.5) (layer F.Cu) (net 10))
 (segment (start 143.3 124) (end 143.3 126.195) (width 0.5) (layer F.Cu) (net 11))
 (segment (start 143.29 126.63) (end 142.24 127.68) (width 0.5) (layer F.Cu) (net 11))
 (segment (start 143.29 125.8) (end 143.29 126.63) (width 0.5) (layer F.Cu) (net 11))
 (segment (start 143.703002 127.68) (end 143.24 127.68) (width 0.25) (layer F.Cu) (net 11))
 (segment (start 144.725001 128.701999) (end 143.703002 127.68) (width 0.25) (layer F.Cu) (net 11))
 (segment (start 144.725001 135.086411) (end 144.725001 128.701999) (width 0.25) (layer F.Cu) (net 11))
 (segment (start 143.24 127.68) (end 142.24 127.68) (width 0.25) (layer F.Cu) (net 11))
 (segment (start 143.33 136.481412) (end 144.725001 135.086411) (width 0.25) (layer F.Cu) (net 11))
 (segment (start 143.33 138.4) (end 143.33 136.481412) (width 0.25) (layer F.Cu) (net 11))
 (segment (start 146.35 124) (end 146.35 126.285) (width 0.5) (layer F.Cu) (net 1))
 (segment (start 146.35 126.39) (end 147.64 127.68) (width 0.5) (layer F.Cu) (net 1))
 (segment (start 146.35 125.8) (end 146.35 126.39) (width 0.5) (layer F.Cu) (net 1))
 (segment (start 145.87 136.31) (end 145.87 138.4) (width 0.25) (layer F.Cu) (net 1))
 (segment (start 145.17501 135.61501) (end 145.87 136.31) (width 0.25) (layer F.Cu) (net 1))
 (segment (start 146.64 127.68) (end 145.17501 129.14499) (width 0.25) (layer F.Cu) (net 1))
 (segment (start 145.17501 129.14499) (end 145.17501 135.61501) (width 0.25) (layer F.Cu) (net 1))
 (segment (start 147.64 127.68) (end 146.64 127.68) (width 0.25) (layer F.Cu) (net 1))
 (segment (start 147.9 119.516) (end 148.9 119.516) (width 0.25) (layer F.Cu) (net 2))
 (segment (start 149.703201 123.846799) (end 149.55 124) (width 0.5) (layer F.Cu) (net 2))
 (segment (start 149.55 124) (end 148.45 124) (width 0.5) (layer F.Cu) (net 2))
 (segment (start 149.703201 120.743499) (end 149.703201 123.846799) (width 0.5) (layer F.Cu) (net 2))
 (segment (start 148.780502 119.8208) (end 149.703201 120.743499) (width 0.5) (layer F.Cu) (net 2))
 (segment (start 148.5032 119.8208) (end 148.780502 119.8208) (width 0.5) (layer F.Cu) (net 2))
 (segment (start 148.45 124) (end 148.45 125.8) (width 0.5) (layer F.Cu) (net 2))
 (segment (start 148.284 120.04) (end 148.5032 119.8208) (width 0.5) (layer F.Cu) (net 2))
 (segment (start 145.45 120.04) (end 148.284 120.04) (width 0.5) (layer F.Cu) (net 2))
 (segment (start 148.230002 128.95) (end 147.64 128.95) (width 0.5) (layer F.Cu) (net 2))
 (segment (start 148.840001 128.340001) (end 148.230002 128.95) (width 0.5) (layer F.Cu) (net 2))
 (segment (start 148.840001 126.190001) (end 148.840001 128.340001) (width 0.5) (layer F.Cu) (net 2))
 (segment (start 148.45 125.8) (end 148.840001 126.190001) (width 0.5) (layer F.Cu) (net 2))
 (segment (start 147.522 118.77) (end 148.5032 117.7888) (width 0.5) (layer F.Cu) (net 5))
 (segment (start 146.72 118.77) (end 147.522 118.77) (width 0.5) (layer F.Cu) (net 5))
 (segment (start 148.6309 117.7888) (end 148.5032 117.7888) (width 0.5) (layer F.Cu) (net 5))
 (segment (start 150.403211 124.136752) (end 150.403211 119.561111) (width 0.5) (layer F.Cu) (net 5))
 (segment (start 150.403211 119.561111) (end 148.6309 117.7888) (width 0.5) (layer F.Cu) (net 5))
 (segment (start 149.61 124.929963) (end 150.403211 124.136752) (width 0.5) (layer F.Cu) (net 5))
 (segment (start 149.61 132.6) (end 149.61 124.929963) (width 0.5) (layer F.Cu) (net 5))
 (segment (start 149.63 132.62) (end 149.61 132.6) (width 0.5) (layer F.Cu) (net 5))
 (segment (start 151.58 132.62) (end 149.63 132.62) (width 0.5) (layer F.Cu) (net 5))
 (segment (start 148.18 134.03) (end 147.64 134.03) (width 0.5) (layer F.Cu) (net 5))
 (segment (start 149.61 132.6) (end 148.18 134.03) (width 0.5) (layer F.Cu) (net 5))
 (segment (start 149.63 134.72) (end 149.61 134.7) (width 0.5) (layer F.Cu) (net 6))
 (segment (start 151.58 134.72) (end 149.63 134.72) (width 0.5) (layer F.Cu) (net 6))
 (segment (start 149.01 135.3) (end 147.64 135.3) (width 0.5) (layer F.Cu) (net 6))
 (segment (start 149.61 134.7) (end 149.01 135.3) (width 0.5) (layer F.Cu) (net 6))
 (segment (start 148.64 135.3) (end 147.64 135.3) (width 0.25) (layer F.Cu) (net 6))
 (segment (start 149.05 135.3) (end 148.64 135.3) (width 0.25) (layer F.Cu) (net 6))
 (segment (start 150.95 137.2) (end 149.05 135.3) (width 0.25) (layer F.Cu) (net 6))
 (segment (start 150.95 138.4) (end 150.95 137.2) (width 0.25) (layer F.Cu) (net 6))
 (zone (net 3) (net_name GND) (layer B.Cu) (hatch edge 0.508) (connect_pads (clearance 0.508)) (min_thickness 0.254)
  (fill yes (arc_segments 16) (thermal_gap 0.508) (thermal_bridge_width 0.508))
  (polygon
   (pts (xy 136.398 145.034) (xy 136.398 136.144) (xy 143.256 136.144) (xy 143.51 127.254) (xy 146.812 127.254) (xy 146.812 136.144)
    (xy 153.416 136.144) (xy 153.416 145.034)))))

